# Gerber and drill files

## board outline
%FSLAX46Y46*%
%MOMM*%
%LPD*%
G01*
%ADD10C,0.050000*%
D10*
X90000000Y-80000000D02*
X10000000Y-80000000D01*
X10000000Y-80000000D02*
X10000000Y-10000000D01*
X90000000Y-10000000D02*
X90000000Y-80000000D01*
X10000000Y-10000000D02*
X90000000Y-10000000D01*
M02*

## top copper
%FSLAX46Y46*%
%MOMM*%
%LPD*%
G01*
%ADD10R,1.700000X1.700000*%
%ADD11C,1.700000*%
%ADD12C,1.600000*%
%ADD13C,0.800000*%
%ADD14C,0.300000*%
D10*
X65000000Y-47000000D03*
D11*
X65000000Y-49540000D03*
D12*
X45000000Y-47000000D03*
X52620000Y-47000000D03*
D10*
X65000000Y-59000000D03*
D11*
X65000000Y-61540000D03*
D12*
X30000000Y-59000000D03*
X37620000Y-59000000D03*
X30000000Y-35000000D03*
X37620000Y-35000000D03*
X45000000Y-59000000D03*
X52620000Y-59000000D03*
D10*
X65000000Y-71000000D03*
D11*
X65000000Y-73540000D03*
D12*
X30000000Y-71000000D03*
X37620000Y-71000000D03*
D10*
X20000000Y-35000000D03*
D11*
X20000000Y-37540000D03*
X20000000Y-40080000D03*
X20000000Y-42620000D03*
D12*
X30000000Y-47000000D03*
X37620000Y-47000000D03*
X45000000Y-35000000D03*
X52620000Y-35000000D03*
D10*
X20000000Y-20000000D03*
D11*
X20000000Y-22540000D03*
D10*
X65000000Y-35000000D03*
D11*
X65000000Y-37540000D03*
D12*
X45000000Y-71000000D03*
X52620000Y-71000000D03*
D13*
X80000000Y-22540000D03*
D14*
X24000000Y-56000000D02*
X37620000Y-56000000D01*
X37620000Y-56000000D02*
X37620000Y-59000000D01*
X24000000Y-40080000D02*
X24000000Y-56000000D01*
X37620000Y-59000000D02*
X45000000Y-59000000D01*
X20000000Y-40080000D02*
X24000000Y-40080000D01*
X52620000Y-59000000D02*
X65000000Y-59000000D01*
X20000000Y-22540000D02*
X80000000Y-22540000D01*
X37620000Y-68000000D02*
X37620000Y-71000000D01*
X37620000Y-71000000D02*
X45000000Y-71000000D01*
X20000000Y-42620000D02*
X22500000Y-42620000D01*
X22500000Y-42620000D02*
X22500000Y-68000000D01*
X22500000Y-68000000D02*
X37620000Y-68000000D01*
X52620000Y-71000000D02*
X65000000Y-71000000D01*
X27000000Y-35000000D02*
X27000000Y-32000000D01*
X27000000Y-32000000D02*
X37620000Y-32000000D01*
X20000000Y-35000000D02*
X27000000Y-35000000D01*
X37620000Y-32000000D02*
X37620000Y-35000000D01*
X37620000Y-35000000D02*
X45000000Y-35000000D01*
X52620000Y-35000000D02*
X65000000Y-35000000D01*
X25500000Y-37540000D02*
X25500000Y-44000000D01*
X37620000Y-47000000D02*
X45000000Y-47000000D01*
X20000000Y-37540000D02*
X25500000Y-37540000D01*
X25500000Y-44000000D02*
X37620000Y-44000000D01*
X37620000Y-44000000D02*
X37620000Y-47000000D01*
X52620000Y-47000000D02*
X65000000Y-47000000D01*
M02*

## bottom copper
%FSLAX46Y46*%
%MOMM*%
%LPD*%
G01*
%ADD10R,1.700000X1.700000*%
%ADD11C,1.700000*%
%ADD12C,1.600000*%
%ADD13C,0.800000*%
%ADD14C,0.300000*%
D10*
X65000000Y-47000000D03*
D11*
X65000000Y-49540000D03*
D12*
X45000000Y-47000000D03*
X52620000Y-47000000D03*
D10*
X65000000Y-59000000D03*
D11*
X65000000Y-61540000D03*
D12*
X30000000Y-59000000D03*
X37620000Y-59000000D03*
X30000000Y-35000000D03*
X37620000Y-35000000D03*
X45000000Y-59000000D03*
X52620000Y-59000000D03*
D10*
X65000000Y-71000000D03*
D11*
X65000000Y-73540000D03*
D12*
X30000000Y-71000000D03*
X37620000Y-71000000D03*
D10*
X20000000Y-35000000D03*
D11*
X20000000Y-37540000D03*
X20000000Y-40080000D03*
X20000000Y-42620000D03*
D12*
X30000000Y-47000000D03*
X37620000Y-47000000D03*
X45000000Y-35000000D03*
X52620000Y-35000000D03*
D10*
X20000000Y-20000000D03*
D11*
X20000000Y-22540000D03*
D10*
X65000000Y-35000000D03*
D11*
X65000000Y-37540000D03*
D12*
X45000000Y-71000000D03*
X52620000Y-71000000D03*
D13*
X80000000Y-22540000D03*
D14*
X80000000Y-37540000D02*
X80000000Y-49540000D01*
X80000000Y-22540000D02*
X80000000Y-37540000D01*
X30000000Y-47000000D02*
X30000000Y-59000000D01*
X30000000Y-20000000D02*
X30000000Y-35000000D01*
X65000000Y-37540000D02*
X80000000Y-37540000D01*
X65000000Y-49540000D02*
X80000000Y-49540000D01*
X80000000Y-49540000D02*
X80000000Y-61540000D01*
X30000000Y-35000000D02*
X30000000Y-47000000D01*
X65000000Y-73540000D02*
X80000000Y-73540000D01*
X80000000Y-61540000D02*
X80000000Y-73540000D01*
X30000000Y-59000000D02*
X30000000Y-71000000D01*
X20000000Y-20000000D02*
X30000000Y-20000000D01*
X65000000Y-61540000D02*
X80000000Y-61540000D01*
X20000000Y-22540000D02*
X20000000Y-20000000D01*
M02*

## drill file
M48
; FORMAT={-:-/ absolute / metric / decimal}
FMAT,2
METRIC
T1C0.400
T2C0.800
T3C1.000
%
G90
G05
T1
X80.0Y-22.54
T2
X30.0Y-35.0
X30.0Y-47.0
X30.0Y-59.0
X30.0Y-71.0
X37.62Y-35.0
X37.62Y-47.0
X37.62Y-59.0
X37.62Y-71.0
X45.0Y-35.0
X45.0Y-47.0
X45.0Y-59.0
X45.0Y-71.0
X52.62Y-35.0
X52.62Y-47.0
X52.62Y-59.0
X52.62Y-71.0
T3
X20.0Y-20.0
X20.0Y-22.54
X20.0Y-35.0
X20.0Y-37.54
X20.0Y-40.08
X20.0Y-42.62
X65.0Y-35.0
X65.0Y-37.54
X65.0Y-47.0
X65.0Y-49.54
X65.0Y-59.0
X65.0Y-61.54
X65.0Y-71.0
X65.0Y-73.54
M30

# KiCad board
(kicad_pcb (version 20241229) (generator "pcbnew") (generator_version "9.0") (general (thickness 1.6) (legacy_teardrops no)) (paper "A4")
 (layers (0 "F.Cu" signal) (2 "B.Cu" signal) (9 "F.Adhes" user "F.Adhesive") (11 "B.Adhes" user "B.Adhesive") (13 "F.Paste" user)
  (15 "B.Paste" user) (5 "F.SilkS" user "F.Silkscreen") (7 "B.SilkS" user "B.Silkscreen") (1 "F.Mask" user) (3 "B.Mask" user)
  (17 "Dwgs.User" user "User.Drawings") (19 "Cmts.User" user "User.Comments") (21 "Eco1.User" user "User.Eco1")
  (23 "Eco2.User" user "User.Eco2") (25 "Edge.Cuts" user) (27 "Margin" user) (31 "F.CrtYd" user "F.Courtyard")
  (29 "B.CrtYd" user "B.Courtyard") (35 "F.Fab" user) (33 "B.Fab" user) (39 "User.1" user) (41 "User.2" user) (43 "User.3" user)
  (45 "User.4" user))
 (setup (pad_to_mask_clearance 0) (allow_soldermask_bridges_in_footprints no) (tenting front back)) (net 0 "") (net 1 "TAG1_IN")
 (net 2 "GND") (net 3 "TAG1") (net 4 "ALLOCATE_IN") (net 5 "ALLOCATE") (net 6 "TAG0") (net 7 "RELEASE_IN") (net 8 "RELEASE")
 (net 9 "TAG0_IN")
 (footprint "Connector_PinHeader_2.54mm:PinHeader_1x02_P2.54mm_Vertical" (layer "F.Cu") (at 65 47)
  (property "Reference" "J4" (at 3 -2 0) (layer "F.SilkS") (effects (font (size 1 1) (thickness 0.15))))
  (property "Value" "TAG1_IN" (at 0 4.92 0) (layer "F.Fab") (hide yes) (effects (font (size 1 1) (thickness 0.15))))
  (pad "1" thru_hole rect (at 0 0) (size 1.7 1.7) (drill 1) (layers "*.Cu" "*.Mask") (remove_unused_layers no) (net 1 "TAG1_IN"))
  (pad "2" thru_hole circle (at 0 2.54) (size 1.7 1.7) (drill 1) (layers "*.Cu" "*.Mask") (remove_unused_layers no) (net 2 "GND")))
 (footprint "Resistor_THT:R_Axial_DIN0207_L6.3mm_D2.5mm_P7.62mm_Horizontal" (layer "F.Cu") (at 45 47)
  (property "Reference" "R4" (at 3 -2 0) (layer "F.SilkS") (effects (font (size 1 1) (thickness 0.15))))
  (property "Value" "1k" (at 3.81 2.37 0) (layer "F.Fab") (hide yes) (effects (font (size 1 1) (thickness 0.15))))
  (pad "1" thru_hole circle (at 0 0) (size 1.6 1.6) (drill 0.8) (layers "*.Cu" "*.Mask") (remove_unused_layers no) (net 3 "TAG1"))
  (pad "2" thru_hole circle (at 7.62 0) (size 1.6 1.6) (drill 0.8) (layers "*.Cu" "*.Mask") (remove_unused_layers no) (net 1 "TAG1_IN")))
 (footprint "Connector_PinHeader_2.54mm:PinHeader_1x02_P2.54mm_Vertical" (layer "F.Cu") (at 65 59)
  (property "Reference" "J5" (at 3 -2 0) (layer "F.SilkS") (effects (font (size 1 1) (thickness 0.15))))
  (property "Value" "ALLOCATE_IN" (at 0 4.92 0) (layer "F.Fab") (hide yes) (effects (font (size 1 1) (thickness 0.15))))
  (pad "1" thru_hole rect (at 0 0) (size 1.7 1.7) (drill 1) (layers "*.Cu" "*.Mask") (remove_unused_layers no) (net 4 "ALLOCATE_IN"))
  (pad "2" thru_hole circle (at 0 2.54) (size 1.7 1.7) (drill 1) (layers "*.Cu" "*.Mask") (remove_unused_layers no) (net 2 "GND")))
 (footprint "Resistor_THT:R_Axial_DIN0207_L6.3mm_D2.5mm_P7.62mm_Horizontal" (layer "F.Cu") (at 30 59)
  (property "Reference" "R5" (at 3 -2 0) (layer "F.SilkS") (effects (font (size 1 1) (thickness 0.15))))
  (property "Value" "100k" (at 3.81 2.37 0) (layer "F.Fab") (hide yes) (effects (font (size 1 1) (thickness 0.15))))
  (pad "1" thru_hole circle (at 0 0) (size 1.6 1.6) (drill 0.8) (layers "*.Cu" "*.Mask") (remove_unused_layers no) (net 2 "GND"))
  (pad "2" thru_hole circle (at 7.62 0) (size 1.6 1.6) (drill 0.8) (layers "*.Cu" "*.Mask") (remove_unused_layers no) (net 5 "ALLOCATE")))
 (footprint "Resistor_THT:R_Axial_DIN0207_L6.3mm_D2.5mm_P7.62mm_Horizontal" (layer "F.Cu") (at 30 35)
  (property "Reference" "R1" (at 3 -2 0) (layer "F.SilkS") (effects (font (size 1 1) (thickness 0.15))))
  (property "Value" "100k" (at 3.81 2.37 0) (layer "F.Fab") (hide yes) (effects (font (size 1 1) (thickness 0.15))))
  (pad "1" thru_hole circle (at 0 0) (size 1.6 1.6) (drill 0.8) (layers "*.Cu" "*.Mask") (remove_unused_layers no) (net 2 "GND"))
  (pad "2" thru_hole circle (at 7.62 0) (size 1.6 1.6) (drill 0.8) (layers "*.Cu" "*.Mask") (remove_unused_layers no) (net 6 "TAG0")))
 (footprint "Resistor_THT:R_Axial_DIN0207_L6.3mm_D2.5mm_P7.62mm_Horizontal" (layer "F.Cu") (at 45 59)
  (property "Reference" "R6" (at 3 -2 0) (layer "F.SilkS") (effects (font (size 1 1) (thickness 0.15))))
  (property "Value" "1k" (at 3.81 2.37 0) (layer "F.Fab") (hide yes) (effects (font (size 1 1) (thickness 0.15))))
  (pad "1" thru_hole circle (at 0 0) (size 1.6 1.6) (drill 0.8) (layers "*.Cu" "*.Mask") (remove_unused_layers no) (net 5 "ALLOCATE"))
  (pad "2" thru_hole circle (at 7.62 0) (size 1.6 1.6) (drill 0.8) (layers "*.Cu" "*.Mask") (remove_unused_layers no) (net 4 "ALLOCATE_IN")))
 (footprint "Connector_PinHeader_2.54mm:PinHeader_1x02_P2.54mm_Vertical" (layer "F.Cu") (at 65 71)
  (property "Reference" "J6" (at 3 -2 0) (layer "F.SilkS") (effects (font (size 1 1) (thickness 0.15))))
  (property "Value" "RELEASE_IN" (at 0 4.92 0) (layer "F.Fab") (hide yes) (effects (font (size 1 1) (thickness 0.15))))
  (pad "1" thru_hole rect (at 0 0) (size 1.7 1.7) (drill 1) (layers "*.Cu" "*.Mask") (remove_unused_layers no) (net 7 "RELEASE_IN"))
  (pad "2" thru_hole circle (at 0 2.54) (size 1.7 1.7) (drill 1) (layers "*.Cu" "*.Mask") (remove_unused_layers no) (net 2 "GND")))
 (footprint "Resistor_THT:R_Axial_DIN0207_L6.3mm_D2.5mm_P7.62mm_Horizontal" (layer "F.Cu") (at 30 71)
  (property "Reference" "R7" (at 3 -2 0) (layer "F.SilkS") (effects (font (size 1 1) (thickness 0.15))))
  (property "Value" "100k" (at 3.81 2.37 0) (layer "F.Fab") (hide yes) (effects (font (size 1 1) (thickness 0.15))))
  (pad "1" thru_hole circle (at 0 0) (size 1.6 1.6) (drill 0.8) (layers "*.Cu" "*.Mask") (remove_unused_layers no) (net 2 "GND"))
  (pad "2" thru_hole circle (at 7.62 0) (size 1.6 1.6) (drill 0.8) (layers "*.Cu" "*.Mask") (remove_unused_layers no) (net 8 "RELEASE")))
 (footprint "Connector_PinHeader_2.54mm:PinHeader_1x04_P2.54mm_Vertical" (layer "F.Cu") (at 20 35)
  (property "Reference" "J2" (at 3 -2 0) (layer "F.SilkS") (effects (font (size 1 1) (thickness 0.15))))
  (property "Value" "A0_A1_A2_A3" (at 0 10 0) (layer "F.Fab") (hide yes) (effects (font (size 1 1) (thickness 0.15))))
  (pad "1" thru_hole rect (at 0 0) (size 1.7 1.7) (drill 1) (layers "*.Cu" "*.Mask") (remove_unused_layers no) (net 6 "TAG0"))
  (pad "2" thru_hole circle (at 0 2.54) (size 1.7 1.7) (drill 1) (layers "*.Cu" "*.Mask") (remove_unused_layers no) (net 3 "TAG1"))
  (pad "3" thru_hole circle (at 0 5.08) (size 1.7 1.7) (drill 1) (layers "*.Cu" "*.Mask") (remove_unused_layers no) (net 5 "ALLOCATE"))
  (pad "4" thru_hole circle (at 0 7.62) (size 1.7 1.7) (drill 1) (layers "*.Cu" "*.Mask") (remove_unused_layers no) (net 8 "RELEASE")))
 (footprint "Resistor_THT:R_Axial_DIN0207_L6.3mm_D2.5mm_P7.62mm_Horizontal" (layer "F.Cu") (at 30 47)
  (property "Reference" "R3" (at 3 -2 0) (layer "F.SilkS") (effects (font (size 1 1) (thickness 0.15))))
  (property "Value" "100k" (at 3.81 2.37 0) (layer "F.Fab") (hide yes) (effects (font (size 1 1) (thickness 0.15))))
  (pad "1" thru_hole circle (at 0 0) (size 1.6 1.6) (drill 0.8) (layers "*.Cu" "*.Mask") (remove_unused_layers no) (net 2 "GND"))
  (pad "2" thru_hole circle (at 7.62 0) (size 1.6 1.6) (drill 0.8) (layers "*.Cu" "*.Mask") (remove_unused_layers no) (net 3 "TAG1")))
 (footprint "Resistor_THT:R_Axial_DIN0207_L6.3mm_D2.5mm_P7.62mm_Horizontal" (layer "F.Cu") (at 45 35)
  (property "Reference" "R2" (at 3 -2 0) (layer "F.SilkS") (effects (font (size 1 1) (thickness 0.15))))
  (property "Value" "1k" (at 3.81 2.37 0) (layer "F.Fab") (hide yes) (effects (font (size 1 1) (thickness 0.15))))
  (pad "1" thru_hole circle (at 0 0) (size 1.6 1.6) (drill 0.8) (layers "*.Cu" "*.Mask") (remove_unused_layers no) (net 6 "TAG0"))
  (pad "2" thru_hole circle (at 7.62 0) (size 1.6 1.6) (drill 0.8) (layers "*.Cu" "*.Mask") (remove_unused_layers no) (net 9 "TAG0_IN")))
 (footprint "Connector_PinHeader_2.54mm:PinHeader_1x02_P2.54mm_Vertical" (layer "F.Cu") (at 20 20)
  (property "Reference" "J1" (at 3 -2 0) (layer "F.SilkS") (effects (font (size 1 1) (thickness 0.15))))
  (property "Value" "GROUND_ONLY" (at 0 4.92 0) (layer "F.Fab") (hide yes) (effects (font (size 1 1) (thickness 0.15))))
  (pad "1" thru_hole rect (at 0 0) (size 1.7 1.7) (drill 1) (layers "*.Cu" "*.Mask") (remove_unused_layers no) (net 2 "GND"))
  (pad "2" thru_hole circle (at 0 2.54) (size 1.7 1.7) (drill 1) (layers "*.Cu" "*.Mask") (remove_unused_layers no) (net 2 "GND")))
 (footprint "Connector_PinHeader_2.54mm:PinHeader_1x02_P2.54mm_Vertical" (layer "F.Cu") (at 65 35)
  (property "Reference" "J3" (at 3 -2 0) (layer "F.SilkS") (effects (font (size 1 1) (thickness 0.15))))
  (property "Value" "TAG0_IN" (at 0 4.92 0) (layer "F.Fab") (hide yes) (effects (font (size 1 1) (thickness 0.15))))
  (pad "1" thru_hole rect (at 0 0) (size 1.7 1.7) (drill 1) (layers "*.Cu" "*.Mask") (remove_unused_layers no) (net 9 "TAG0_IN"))
  (pad "2" thru_hole circle (at 0 2.54) (size 1.7 1.7) (drill 1) (layers "*.Cu" "*.Mask") (remove_unused_layers no) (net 2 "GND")))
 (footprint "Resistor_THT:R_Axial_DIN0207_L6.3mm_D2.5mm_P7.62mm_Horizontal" (layer "F.Cu") (at 45 71)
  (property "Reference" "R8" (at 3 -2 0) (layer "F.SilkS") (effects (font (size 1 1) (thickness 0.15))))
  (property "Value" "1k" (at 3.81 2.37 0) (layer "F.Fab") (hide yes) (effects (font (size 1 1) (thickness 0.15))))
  (pad "1" thru_hole circle (at 0 0) (size 1.6 1.6) (drill 0.8) (layers "*.Cu" "*.Mask") (remove_unused_layers no) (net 8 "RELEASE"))
  (pad "2" thru_hole circle (at 7.62 0) (size 1.6 1.6) (drill 0.8) (layers "*.Cu" "*.Mask") (remove_unused_layers no) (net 7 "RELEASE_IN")))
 (gr_line (start 90 80) (end 10 80) (stroke (width 0.05) (type default)) (layer "Edge.Cuts"))
 (gr_line (start 10 80) (end 10 10) (stroke (width 0.05) (type default)) (layer "Edge.Cuts"))
 (gr_line (start 90 10) (end 90 80) (stroke (width 0.05) (type default)) (layer "Edge.Cuts"))
 (gr_line (start 10 10) (end 90 10) (stroke (width 0.05) (type default)) (layer "Edge.Cuts"))
 (segment (start 24 56) (end 37.62 56) (width 0.3) (layer "F.Cu") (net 5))
 (segment (start 37.62 56) (end 37.62 59) (width 0.3) (layer "F.Cu") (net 5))
 (segment (start 24 40.08) (end 24 56) (width 0.3) (layer "F.Cu") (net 5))
 (segment (start 37.62 59) (end 45 59) (width 0.3) (layer "F.Cu") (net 5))
 (segment (start 20 40.08) (end 24 40.08) (width 0.3) (layer "F.Cu") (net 5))
 (segment (start 52.62 59) (end 65 59) (width 0.3) (layer "F.Cu") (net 4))
 (segment (start 20 22.54) (end 80 22.54) (width 0.3) (layer "F.Cu") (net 2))
 (via (at 80 22.54) (size 0.8) (drill 0.4) (layers "F.Cu" "B.Cu") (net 2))
 (segment (start 80 37.54) (end 80 49.54) (width 0.3) (layer "B.Cu") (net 2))
 (segment (start 80 22.54) (end 80 37.54) (width 0.3) (layer "B.Cu") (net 2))
 (segment (start 30 47) (end 30 59) (width 0.3) (layer "B.Cu") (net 2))
 (segment (start 30 20) (end 30 35) (width 0.3) (layer "B.Cu") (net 2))
 (segment (start 65 37.54) (end 80 37.54) (width 0.3) (layer "B.Cu") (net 2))
 (segment (start 65 49.54) (end 80 49.54) (width 0.3) (layer "B.Cu") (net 2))
 (segment (start 80 49.54) (end 80 61.54) (width 0.3) (layer "B.Cu") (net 2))
 (segment (start 30 35) (end 30 47) (width 0.3) (layer "B.Cu") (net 2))
 (segment (start 65 73.54) (end 80 73.54) (width 0.3) (layer "B.Cu") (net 2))
 (segment (start 80 61.54) (end 80 73.54) (width 0.3) (layer "B.Cu") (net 2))
 (segment (start 30 59) (end 30 71) (width 0.3) (layer "B.Cu") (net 2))
 (segment (start 20 20) (end 30 20) (width 0.3) (layer "B.Cu") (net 2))
 (segment (start 65 61.54) (end 80 61.54) (width 0.3) (layer "B.Cu") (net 2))
 (segment (start 20 22.54) (end 20 20) (width 0.3) (layer "B.Cu") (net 2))
 (segment (start 37.62 68) (end 37.62 71) (width 0.3) (layer "F.Cu") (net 8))
 (segment (start 37.62 71) (end 45 71) (width 0.3) (layer "F.Cu") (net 8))
 (segment (start 20 42.62) (end 22.5 42.62) (width 0.3) (layer "F.Cu") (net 8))
 (segment (start 22.5 42.62) (end 22.5 68) (width 0.3) (layer "F.Cu") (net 8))
 (segment (start 22.5 68) (end 37.62 68) (width 0.3) (layer "F.Cu") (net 8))
 (segment (start 52.62 71) (end 65 71) (width 0.3) (layer "F.Cu") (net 7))
 (segment (start 27 35) (end 27 32) (width 0.3) (layer "F.Cu") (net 6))
 (segment (start 27 32) (end 37.62 32) (width 0.3) (layer "F.Cu") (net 6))
 (segment (start 20 35) (end 27 35) (width 0.3) (layer "F.Cu") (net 6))
 (segment (start 37.62 32) (end 37.62 35) (width 0.3) (layer "F.Cu") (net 6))
 (segment (start 37.62 35) (end 45 35) (width 0.3) (layer "F.Cu") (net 6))
 (segment (start 52.62 35) (end 65 35) (width 0.3) (layer "F.Cu") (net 9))
 (segment (start 25.5 37.54) (end 25.5 44) (width 0.3) (layer "F.Cu") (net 3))
 (segment (start 37.62 47) (end 45 47) (width 0.3) (layer "F.Cu") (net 3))
 (segment (start 20 37.54) (end 25.5 37.54) (width 0.3) (layer "F.Cu") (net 3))
 (segment (start 25.5 44) (end 37.62 44) (width 0.3) (layer "F.Cu") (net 3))
 (segment (start 37.62 44) (end 37.62 47) (width 0.3) (layer "F.Cu") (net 3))
 (segment (start 52.62 47) (end 65 47) (width 0.3) (layer "F.Cu") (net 1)))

